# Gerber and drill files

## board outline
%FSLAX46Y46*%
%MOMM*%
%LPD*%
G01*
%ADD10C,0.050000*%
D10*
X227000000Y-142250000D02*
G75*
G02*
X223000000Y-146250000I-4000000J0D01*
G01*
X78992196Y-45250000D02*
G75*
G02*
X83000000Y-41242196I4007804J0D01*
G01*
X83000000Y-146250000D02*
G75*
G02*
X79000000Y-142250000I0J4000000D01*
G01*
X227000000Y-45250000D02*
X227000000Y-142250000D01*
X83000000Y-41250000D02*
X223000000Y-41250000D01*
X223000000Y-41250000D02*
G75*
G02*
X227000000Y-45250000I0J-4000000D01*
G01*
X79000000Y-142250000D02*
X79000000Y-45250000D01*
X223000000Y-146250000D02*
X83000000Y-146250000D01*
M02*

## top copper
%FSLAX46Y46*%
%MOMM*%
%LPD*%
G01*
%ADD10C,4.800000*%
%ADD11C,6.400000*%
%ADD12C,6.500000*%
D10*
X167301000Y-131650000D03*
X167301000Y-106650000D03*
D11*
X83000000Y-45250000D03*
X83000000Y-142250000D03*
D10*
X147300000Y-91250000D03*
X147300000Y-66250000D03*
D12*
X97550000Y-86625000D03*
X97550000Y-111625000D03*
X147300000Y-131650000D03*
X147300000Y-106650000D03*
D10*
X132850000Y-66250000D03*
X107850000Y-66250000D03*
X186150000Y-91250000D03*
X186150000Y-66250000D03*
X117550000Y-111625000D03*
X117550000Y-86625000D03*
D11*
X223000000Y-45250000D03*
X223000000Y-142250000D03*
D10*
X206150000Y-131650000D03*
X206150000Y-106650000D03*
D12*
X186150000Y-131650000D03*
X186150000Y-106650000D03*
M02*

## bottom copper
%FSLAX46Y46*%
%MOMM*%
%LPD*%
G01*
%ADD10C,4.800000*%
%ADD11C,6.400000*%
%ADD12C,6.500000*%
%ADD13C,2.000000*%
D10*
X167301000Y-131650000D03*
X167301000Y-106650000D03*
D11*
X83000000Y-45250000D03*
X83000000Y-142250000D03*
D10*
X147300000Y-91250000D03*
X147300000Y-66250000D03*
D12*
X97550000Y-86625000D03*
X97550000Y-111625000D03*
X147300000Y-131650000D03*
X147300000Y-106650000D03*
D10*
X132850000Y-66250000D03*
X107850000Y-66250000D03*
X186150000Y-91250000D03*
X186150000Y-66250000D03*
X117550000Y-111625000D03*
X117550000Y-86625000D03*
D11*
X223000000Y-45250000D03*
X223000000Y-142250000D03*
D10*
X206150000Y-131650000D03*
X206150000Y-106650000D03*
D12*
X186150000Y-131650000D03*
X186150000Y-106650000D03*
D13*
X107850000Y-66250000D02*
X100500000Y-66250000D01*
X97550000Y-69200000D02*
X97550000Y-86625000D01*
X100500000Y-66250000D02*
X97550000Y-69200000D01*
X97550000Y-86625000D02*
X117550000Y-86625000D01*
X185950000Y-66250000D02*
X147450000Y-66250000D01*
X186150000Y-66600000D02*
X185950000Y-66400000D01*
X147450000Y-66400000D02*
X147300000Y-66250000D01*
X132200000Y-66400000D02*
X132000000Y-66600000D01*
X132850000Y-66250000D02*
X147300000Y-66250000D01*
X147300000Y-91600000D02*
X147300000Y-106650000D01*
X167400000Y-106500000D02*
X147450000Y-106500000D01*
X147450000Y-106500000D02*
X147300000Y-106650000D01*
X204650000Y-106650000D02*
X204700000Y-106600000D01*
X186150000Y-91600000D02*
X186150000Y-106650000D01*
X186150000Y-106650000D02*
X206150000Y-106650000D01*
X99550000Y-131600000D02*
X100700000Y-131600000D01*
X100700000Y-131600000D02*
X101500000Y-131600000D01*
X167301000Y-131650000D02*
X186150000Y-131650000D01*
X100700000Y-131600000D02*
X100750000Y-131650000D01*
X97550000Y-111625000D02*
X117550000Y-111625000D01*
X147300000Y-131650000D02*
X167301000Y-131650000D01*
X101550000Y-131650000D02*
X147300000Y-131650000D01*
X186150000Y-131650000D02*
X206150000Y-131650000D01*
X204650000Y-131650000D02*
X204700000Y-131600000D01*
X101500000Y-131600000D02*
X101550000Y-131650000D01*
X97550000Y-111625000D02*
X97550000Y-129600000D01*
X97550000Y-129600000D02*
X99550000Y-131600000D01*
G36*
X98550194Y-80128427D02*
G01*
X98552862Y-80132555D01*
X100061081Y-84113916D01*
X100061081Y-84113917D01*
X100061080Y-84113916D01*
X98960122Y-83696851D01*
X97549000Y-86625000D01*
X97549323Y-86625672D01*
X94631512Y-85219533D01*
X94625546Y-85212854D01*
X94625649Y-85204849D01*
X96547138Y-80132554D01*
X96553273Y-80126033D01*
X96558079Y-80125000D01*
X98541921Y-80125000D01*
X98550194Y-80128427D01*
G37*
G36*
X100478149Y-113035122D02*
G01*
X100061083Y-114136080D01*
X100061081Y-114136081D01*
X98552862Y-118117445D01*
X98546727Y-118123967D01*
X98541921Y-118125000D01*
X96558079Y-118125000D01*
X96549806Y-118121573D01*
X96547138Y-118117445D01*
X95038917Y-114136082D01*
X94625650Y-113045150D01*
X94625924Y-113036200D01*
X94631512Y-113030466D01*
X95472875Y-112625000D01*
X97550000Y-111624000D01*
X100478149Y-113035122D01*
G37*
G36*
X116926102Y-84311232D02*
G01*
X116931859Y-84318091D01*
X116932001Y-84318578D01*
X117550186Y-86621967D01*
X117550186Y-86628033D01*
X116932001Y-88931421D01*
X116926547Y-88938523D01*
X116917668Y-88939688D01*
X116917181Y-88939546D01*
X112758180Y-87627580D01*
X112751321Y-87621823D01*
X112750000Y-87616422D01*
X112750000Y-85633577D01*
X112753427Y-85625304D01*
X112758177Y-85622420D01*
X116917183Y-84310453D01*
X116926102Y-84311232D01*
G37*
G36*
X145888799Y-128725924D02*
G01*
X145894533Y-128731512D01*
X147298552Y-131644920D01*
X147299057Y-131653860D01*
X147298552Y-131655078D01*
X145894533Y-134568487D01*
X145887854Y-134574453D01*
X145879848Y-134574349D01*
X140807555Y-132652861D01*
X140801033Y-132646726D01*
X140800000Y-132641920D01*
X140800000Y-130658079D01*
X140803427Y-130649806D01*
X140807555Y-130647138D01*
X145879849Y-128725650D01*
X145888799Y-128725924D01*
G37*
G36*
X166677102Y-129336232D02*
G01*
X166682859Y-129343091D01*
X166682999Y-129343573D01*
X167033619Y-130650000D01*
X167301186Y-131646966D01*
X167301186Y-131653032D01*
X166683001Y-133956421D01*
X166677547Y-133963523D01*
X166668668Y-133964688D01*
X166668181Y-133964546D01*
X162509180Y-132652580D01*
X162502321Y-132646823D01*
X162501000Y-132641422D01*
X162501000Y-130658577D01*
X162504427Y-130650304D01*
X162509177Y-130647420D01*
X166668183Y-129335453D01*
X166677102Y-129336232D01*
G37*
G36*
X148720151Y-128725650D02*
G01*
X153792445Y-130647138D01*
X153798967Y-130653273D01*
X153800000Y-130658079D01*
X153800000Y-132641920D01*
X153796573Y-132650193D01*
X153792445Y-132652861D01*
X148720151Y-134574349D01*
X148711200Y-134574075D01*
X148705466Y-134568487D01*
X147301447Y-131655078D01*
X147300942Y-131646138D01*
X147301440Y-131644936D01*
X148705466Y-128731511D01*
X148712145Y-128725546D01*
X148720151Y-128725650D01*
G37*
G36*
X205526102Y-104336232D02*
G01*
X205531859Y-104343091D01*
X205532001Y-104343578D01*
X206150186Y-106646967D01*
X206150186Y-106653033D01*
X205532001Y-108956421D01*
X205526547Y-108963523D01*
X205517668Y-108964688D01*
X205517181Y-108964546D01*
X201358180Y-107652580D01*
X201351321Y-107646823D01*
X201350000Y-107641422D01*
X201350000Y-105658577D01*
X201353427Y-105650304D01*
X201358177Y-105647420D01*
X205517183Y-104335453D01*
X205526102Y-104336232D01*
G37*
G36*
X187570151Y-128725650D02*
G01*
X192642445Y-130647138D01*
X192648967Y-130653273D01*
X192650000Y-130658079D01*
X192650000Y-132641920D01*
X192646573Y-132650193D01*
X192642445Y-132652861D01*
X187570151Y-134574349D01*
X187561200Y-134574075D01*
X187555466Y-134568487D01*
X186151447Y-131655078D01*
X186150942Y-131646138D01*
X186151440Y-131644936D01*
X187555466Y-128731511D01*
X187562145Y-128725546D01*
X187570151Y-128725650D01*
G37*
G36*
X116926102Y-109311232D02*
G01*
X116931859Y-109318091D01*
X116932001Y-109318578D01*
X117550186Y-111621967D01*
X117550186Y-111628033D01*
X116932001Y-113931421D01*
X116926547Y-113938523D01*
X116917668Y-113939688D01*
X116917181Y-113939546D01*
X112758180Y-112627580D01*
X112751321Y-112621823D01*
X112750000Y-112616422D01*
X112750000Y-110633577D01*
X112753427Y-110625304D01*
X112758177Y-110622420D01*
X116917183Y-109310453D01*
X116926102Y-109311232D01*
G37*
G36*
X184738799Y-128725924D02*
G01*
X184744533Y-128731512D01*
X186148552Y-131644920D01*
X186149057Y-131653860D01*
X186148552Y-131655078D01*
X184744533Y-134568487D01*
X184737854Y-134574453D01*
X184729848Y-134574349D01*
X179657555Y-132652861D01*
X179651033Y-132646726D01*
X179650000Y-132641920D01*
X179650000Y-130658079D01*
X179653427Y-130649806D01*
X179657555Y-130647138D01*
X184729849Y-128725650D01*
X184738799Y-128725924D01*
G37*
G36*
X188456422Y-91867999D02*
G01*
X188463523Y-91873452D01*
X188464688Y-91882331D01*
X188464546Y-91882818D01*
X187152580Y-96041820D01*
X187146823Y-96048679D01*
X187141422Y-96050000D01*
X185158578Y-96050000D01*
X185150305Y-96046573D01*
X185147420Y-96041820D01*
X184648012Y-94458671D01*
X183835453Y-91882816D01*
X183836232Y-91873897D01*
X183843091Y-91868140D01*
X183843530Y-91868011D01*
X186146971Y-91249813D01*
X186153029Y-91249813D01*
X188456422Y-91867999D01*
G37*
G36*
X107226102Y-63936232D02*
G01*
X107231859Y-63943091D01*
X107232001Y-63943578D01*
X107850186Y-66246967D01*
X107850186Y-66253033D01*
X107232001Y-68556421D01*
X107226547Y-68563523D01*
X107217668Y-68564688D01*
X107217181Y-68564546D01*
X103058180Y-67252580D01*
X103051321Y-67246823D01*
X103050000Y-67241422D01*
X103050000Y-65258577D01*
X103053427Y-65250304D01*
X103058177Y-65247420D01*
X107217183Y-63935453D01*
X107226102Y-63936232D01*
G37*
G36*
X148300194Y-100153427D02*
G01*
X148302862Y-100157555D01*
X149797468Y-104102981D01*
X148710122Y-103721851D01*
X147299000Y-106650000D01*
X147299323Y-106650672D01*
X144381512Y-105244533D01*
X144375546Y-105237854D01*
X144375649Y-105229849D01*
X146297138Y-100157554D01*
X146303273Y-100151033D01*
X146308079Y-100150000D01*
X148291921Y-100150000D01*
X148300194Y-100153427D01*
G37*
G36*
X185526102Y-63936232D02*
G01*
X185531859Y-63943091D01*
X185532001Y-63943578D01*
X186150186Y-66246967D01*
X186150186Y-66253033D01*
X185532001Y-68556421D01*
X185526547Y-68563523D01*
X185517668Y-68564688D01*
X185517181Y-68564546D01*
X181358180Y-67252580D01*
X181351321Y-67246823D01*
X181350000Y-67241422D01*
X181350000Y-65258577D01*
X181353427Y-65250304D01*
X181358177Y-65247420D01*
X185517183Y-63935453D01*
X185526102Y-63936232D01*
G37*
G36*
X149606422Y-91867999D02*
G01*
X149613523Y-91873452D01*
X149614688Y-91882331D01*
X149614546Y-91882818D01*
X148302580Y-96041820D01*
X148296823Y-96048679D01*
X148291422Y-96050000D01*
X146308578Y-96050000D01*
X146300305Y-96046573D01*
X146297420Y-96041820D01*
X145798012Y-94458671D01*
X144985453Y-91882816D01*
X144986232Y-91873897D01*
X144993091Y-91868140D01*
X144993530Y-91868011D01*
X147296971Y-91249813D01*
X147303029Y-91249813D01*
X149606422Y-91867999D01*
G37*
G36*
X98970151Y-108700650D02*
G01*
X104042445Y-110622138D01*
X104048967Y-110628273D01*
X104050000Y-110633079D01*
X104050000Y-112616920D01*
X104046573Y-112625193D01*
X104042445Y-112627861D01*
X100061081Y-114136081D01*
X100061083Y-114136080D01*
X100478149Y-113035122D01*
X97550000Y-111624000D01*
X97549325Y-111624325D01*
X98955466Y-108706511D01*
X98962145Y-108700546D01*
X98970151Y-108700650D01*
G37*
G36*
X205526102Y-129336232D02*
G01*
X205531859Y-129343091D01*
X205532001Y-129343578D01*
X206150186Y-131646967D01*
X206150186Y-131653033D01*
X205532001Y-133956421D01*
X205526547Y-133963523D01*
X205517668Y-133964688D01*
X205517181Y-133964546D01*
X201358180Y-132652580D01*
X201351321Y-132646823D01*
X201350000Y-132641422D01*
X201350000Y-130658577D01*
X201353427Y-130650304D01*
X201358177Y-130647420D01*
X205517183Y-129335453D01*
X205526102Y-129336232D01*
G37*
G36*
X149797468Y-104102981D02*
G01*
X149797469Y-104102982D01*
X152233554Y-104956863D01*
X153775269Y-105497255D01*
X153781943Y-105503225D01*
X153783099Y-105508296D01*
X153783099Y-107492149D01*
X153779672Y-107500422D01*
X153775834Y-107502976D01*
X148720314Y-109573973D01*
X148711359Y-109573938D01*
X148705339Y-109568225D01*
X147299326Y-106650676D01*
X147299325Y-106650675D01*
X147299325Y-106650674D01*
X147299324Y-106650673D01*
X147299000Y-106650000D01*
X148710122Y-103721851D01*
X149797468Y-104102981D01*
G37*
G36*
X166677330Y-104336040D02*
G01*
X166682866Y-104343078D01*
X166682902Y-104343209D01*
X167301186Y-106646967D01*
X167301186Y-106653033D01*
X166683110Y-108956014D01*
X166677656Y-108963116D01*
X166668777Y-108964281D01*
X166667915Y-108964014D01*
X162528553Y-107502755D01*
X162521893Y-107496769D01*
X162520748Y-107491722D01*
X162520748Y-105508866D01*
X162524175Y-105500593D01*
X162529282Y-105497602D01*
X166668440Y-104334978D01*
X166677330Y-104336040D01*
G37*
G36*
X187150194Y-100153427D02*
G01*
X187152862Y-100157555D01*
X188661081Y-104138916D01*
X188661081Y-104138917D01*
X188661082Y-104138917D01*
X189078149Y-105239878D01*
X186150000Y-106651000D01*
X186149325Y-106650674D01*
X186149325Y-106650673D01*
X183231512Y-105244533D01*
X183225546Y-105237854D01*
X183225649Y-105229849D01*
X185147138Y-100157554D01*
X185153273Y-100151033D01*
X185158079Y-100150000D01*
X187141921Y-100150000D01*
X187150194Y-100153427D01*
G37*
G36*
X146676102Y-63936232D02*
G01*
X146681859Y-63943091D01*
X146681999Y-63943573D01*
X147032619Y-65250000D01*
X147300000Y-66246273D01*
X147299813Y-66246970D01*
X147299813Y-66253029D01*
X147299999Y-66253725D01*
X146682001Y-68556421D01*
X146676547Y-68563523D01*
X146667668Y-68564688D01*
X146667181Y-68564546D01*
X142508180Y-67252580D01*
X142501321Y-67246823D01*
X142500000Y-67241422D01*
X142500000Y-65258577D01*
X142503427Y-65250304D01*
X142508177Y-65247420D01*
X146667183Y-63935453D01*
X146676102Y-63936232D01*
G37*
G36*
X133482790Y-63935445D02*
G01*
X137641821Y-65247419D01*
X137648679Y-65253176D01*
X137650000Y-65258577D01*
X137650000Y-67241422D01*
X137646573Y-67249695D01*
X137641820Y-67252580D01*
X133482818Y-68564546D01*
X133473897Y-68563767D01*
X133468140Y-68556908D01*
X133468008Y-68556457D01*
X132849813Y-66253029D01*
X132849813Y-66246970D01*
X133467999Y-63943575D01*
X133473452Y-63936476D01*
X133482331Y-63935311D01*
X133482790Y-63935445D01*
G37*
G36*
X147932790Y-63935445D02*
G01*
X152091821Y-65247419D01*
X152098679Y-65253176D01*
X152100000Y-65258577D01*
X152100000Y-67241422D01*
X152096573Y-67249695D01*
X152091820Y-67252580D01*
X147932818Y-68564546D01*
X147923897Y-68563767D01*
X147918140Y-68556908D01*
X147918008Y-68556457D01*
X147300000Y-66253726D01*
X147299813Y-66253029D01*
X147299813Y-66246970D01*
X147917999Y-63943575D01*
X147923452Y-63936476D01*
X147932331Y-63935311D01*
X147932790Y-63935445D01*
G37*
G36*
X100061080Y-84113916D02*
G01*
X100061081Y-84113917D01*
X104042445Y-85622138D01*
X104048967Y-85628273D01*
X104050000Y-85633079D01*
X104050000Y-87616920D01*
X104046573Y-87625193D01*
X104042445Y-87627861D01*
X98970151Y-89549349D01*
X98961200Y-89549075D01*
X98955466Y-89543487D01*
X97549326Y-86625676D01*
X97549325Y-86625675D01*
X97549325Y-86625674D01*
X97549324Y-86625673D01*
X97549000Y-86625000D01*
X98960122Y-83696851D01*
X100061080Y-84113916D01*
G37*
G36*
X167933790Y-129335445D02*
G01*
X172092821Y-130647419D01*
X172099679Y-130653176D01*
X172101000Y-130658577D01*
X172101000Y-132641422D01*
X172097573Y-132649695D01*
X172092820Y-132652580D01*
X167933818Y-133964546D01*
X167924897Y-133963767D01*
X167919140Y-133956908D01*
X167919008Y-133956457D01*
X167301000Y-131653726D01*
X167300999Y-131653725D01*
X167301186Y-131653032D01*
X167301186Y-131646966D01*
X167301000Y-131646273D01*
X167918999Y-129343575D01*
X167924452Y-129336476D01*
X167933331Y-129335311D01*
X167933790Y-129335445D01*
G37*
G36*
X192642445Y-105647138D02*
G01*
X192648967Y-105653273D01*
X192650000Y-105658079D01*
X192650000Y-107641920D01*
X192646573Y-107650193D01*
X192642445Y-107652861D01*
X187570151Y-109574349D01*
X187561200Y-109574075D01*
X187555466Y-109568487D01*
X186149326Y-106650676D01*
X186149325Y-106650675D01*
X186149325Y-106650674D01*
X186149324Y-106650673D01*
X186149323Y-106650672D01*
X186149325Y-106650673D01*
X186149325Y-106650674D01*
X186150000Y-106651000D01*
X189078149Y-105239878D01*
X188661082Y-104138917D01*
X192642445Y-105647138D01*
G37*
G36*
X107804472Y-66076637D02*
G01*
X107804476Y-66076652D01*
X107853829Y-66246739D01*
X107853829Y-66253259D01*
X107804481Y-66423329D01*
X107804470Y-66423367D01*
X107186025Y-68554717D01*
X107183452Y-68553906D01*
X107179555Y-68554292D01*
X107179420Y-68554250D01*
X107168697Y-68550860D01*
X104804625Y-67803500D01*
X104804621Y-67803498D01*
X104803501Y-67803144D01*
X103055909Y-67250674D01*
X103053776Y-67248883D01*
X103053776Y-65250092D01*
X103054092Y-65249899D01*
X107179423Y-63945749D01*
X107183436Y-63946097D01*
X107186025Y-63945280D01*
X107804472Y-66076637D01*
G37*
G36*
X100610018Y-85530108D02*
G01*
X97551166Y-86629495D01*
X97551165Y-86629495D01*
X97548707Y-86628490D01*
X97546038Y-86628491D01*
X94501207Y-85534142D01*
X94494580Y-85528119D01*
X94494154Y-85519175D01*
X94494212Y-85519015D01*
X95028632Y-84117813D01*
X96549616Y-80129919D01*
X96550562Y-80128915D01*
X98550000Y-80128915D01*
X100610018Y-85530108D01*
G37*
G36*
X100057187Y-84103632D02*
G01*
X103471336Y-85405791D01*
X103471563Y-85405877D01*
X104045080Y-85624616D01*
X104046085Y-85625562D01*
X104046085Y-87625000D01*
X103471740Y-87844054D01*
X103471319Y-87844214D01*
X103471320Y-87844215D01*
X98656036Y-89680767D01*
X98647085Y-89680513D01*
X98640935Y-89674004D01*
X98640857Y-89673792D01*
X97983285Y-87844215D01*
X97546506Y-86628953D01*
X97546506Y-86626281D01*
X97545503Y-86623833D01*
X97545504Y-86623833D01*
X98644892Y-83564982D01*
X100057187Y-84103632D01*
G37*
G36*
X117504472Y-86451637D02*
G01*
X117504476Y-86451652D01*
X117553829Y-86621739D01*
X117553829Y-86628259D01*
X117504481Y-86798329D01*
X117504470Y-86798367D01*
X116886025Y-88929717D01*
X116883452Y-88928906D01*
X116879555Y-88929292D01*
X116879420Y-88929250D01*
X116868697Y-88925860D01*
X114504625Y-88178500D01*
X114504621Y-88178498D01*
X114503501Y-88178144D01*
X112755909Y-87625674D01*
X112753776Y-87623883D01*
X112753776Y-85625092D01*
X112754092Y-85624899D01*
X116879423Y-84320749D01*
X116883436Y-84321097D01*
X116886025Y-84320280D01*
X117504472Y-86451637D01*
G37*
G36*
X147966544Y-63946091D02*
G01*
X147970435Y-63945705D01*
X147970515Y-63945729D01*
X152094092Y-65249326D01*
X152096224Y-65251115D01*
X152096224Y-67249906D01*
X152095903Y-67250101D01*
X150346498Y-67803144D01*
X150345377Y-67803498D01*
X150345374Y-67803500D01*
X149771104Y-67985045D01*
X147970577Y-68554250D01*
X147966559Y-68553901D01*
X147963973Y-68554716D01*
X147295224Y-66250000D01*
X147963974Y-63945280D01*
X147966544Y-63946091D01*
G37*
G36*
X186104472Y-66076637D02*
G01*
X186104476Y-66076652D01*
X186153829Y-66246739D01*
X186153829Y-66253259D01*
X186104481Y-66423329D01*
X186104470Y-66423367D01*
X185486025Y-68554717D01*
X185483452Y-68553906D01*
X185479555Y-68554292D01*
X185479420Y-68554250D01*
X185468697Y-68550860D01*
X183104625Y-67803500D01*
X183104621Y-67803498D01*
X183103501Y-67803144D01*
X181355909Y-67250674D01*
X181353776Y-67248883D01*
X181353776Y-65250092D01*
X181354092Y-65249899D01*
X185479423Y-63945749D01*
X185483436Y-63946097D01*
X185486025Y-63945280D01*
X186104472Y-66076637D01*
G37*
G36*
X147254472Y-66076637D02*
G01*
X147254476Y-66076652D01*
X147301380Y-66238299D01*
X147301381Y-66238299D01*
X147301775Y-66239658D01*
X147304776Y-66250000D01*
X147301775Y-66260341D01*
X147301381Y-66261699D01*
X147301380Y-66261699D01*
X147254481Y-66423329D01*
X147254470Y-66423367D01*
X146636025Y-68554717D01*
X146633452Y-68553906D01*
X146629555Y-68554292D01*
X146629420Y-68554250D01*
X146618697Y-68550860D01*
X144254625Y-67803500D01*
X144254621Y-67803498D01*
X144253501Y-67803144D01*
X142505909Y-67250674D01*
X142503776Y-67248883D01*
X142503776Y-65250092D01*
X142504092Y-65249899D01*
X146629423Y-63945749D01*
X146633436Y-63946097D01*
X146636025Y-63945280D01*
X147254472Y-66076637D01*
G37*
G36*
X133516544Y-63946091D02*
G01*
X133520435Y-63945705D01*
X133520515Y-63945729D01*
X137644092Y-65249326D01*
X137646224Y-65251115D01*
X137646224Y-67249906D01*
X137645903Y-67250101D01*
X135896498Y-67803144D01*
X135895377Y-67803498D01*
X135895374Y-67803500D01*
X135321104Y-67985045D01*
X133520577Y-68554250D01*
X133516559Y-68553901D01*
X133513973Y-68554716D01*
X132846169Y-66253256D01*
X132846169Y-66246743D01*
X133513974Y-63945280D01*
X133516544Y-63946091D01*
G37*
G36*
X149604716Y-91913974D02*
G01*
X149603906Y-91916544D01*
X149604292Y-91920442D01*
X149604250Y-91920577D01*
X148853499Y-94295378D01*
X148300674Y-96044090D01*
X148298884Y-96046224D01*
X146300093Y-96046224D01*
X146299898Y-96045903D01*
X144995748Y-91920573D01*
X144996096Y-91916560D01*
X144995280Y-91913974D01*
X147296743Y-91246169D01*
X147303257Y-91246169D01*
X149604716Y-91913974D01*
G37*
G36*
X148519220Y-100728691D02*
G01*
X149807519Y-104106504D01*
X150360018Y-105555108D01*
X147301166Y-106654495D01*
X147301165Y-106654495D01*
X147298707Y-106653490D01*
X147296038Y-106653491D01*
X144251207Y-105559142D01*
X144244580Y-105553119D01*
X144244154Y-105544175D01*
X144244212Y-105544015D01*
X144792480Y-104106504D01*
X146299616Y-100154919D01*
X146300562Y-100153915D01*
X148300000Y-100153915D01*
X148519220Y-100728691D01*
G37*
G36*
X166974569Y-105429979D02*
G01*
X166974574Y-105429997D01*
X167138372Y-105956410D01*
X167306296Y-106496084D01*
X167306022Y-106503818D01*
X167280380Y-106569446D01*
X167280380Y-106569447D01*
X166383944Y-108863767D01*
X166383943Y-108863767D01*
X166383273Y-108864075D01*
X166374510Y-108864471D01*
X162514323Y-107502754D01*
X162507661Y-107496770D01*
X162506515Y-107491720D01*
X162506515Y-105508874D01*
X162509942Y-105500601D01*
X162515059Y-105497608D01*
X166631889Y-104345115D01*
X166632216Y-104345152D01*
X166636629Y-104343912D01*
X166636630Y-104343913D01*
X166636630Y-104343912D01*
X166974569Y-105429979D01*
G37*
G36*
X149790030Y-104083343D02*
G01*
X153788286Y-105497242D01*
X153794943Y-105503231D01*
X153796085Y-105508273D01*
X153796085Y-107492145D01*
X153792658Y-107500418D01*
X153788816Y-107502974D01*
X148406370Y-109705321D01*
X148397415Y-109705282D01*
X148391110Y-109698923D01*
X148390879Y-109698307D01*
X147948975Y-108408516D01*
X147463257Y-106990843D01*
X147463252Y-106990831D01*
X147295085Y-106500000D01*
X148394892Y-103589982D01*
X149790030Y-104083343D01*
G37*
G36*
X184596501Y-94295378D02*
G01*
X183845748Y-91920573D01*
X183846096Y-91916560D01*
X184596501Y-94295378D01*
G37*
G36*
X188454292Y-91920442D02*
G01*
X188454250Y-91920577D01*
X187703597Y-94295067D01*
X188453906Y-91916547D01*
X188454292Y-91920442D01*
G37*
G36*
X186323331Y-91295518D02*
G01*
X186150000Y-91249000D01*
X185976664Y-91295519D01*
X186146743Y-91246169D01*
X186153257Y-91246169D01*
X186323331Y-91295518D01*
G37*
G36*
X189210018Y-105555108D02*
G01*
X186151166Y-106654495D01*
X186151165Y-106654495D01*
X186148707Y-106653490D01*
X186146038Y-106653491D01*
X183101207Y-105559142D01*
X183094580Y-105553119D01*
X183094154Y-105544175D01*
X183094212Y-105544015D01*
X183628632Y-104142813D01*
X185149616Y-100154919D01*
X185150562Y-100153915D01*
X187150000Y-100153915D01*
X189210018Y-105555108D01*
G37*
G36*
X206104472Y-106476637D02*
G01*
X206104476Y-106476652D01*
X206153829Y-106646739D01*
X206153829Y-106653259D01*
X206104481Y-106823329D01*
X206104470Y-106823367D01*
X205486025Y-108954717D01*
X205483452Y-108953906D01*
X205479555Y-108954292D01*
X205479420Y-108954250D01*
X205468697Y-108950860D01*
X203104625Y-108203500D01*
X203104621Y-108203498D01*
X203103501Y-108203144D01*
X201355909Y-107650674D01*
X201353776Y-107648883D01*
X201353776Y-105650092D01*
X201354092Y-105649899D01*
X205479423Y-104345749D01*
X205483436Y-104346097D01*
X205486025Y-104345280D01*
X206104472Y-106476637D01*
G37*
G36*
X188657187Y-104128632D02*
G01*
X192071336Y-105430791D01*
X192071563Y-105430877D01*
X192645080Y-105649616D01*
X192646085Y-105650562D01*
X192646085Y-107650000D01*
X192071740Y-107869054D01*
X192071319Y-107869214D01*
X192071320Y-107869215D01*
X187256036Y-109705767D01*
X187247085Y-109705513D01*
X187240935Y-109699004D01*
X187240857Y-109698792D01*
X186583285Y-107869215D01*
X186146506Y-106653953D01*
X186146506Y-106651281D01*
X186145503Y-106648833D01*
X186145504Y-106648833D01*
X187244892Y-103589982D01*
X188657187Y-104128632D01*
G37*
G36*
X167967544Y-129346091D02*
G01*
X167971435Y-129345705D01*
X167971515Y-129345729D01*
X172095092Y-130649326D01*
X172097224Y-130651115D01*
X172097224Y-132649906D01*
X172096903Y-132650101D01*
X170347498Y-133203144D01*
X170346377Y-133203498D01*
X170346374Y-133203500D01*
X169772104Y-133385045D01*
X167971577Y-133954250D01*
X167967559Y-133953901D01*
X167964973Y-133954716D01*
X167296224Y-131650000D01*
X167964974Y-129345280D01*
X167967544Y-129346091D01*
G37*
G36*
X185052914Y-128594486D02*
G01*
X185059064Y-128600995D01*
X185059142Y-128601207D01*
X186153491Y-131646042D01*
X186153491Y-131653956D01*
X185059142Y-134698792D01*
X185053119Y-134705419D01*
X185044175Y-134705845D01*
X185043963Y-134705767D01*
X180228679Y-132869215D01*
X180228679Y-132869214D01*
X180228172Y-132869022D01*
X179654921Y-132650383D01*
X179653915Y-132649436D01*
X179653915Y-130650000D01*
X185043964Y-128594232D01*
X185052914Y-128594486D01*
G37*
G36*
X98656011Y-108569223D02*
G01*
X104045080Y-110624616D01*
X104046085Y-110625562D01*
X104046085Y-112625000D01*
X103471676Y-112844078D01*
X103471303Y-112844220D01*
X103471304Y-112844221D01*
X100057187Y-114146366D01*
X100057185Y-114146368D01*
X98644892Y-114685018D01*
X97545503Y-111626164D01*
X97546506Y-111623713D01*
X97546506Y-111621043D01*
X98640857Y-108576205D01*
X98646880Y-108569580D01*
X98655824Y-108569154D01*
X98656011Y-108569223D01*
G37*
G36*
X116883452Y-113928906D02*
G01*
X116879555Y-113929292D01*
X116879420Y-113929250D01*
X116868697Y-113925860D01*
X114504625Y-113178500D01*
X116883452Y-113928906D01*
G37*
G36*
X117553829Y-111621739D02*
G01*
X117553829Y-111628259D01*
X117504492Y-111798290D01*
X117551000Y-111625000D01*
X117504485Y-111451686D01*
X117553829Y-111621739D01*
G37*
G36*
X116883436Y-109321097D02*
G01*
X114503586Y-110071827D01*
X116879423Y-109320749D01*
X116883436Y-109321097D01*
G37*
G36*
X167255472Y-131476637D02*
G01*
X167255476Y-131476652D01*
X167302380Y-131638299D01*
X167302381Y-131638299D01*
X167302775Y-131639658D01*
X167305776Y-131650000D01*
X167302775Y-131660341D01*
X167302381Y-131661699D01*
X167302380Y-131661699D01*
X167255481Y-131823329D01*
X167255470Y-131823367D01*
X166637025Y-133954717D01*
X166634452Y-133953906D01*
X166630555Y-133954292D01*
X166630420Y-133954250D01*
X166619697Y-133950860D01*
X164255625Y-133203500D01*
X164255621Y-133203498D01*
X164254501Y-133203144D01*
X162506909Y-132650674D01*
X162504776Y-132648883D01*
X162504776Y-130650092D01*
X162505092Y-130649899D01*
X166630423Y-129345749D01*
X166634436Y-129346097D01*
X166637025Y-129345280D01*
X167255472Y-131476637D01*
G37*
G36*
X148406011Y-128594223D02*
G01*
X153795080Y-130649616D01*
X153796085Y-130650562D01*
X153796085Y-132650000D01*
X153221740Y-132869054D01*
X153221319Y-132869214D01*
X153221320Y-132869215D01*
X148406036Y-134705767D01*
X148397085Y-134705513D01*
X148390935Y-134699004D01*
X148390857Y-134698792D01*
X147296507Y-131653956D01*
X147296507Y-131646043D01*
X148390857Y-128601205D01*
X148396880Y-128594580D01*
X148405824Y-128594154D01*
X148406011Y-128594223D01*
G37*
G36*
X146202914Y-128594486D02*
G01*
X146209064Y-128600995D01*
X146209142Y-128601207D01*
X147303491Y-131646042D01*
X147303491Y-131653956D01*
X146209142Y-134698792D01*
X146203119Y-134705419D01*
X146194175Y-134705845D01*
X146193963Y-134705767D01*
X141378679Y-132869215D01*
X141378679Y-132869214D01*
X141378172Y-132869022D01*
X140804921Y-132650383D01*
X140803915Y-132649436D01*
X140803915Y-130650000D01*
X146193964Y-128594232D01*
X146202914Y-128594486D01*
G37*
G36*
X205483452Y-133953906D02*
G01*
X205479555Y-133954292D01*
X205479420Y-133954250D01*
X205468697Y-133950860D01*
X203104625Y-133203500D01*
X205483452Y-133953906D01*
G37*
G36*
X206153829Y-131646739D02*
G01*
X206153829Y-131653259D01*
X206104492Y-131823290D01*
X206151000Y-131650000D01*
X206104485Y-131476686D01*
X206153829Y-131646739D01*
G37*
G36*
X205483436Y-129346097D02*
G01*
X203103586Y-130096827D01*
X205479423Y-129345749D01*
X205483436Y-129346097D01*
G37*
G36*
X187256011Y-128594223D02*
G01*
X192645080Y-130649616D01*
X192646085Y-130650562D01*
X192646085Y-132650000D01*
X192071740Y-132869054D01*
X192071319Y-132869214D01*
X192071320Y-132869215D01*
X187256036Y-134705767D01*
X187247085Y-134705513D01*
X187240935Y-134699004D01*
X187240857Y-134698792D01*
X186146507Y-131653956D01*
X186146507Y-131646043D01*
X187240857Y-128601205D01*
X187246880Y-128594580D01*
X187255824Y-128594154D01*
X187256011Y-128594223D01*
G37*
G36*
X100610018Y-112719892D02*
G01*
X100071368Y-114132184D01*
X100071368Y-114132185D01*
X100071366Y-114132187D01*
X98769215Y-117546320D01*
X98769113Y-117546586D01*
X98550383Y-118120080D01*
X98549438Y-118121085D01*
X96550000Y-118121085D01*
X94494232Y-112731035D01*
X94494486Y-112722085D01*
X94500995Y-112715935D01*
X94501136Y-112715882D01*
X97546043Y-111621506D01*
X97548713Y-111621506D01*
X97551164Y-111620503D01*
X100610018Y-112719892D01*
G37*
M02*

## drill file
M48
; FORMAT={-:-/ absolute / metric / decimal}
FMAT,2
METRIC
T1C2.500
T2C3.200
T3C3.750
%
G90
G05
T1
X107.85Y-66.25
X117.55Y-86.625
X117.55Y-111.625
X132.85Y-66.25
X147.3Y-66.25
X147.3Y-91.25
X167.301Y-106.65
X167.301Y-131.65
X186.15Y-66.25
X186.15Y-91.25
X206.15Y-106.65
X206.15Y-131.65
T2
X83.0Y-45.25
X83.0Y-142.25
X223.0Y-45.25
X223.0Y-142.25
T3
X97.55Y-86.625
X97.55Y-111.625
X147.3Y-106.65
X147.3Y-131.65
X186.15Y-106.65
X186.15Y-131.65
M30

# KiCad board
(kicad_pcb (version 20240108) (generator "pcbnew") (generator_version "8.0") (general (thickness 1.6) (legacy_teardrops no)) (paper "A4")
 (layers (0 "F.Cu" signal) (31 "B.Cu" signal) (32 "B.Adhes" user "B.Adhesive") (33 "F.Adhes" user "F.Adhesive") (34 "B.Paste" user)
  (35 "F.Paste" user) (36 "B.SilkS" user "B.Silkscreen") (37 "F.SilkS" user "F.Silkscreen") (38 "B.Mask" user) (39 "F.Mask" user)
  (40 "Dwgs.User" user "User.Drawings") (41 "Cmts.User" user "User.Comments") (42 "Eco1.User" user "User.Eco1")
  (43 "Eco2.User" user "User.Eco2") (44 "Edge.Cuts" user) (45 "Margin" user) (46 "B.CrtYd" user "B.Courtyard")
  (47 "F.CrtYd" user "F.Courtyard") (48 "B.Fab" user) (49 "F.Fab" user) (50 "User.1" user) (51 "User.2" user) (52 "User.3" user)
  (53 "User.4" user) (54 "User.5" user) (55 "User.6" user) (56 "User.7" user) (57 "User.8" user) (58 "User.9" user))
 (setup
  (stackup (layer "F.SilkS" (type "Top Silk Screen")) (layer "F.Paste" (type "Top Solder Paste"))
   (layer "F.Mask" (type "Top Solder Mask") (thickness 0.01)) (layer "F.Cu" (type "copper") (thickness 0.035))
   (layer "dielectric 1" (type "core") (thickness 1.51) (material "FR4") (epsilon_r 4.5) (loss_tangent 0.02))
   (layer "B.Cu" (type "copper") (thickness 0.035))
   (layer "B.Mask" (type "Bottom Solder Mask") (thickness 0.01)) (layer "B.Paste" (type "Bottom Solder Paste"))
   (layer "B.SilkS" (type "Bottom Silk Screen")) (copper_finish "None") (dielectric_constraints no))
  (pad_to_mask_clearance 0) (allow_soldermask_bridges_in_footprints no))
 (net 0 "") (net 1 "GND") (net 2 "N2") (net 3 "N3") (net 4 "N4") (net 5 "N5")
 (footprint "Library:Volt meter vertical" (layer "F.Cu") (at 167.301 119.15)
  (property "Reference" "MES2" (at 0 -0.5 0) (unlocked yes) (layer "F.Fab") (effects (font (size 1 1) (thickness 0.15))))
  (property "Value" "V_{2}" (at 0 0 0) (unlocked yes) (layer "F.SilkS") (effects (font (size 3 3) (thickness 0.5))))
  (pad "1" thru_hole circle (at 0 12.5 180) (size 4.8 4.8) (drill 2.5) (layers "*.Cu" "*.Mask") (remove_unused_layers no) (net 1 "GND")
   (teardrops (best_length_ratio 0.5) (max_length 8) (best_width_ratio 1) (max_width 8) (curve_points 0) (filter_ratio 0.9) (enabled yes)
    (allow_two_segments yes) (prefer_zone_connections yes)))
  (pad "2" thru_hole circle (at 0 -12.5 180) (size 4.8 4.8) (drill 2.5) (layers "*.Cu" "*.Mask") (remove_unused_layers no) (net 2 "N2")
   (teardrops (best_length_ratio 0.5) (max_length 8) (best_width_ratio 1) (max_width 8) (curve_points 0) (filter_ratio 0.9) (enabled yes)
    (allow_two_segments yes) (prefer_zone_connections yes))))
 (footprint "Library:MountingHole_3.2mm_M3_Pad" (layer "F.Cu") (at 83 45.25)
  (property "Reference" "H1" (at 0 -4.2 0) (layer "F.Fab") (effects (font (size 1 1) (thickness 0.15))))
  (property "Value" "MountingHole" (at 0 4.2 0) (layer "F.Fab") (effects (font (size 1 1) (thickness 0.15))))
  (pad "1" thru_hole circle (at 0 0) (size 6.4 6.4) (drill 3.2) (layers "*.Cu" "*.Mask") (remove_unused_layers no)))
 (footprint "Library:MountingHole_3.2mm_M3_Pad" (layer "F.Cu") (at 83 142.25)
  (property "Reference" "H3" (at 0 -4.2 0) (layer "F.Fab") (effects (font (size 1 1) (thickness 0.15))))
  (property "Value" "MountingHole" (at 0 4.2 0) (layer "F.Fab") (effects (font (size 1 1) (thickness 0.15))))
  (pad "1" thru_hole circle (at 0 0) (size 6.4 6.4) (drill 3.2) (layers "*.Cu" "*.Mask") (remove_unused_layers no)))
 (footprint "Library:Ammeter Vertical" (layer "F.Cu") (at 147.3 78.75 -90)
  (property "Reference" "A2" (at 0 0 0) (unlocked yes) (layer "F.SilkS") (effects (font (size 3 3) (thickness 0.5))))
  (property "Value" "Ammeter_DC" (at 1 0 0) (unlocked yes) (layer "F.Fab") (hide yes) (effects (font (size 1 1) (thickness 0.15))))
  (pad "1" thru_hole circle (at 12.5 0 180) (size 4.8 4.8) (drill 2.5) (layers "*.Cu" "*.Mask") (remove_unused_layers no) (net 2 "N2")
   (teardrops (best_length_ratio 0.5) (max_length 8) (best_width_ratio 1) (max_width 8) (curve_points 0) (filter_ratio 0.9) (enabled yes)
    (allow_two_segments yes) (prefer_zone_connections yes)))
  (pad "2" thru_hole circle (at -12.5 0 180) (size 4.8 4.8) (drill 2.5) (layers "*.Cu" "*.Mask") (remove_unused_layers no) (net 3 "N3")
   (teardrops (best_length_ratio 0.5) (max_length 8) (best_width_ratio 1) (max_width 8) (curve_points 0) (filter_ratio 0.9) (enabled yes)
    (allow_two_segments yes) (prefer_zone_connections yes))))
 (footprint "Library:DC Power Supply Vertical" (layer "F.Cu") (at 97.55 99.125)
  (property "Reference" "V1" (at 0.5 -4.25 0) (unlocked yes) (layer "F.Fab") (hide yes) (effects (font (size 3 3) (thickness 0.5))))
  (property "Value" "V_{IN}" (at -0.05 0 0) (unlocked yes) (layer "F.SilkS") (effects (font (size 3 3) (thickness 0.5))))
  (pad "1" thru_hole circle (at 0 -12.5) (size 6.5 6.5) (drill 3.75) (layers "*.Cu" "*.Mask") (remove_unused_layers no) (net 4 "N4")
   (teardrops (best_length_ratio 0.5) (max_length 8) (best_width_ratio 1) (max_width 8) (curve_points 0) (filter_ratio 0.9) (enabled yes)
    (allow_two_segments yes) (prefer_zone_connections yes)))
  (pad "2" thru_hole circle (at 0 12.5) (size 6.5 6.5) (drill 3.75) (layers "*.Cu" "*.Mask") (remove_unused_layers no) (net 1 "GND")
   (teardrops (best_length_ratio 0.5) (max_length 8) (best_width_ratio 1) (max_width 8) (curve_points 0) (filter_ratio 0.9) (enabled yes)
    (allow_two_segments yes) (prefer_zone_connections yes))))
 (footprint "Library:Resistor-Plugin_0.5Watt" (layer "F.Cu") (at 147.3 119.15 180)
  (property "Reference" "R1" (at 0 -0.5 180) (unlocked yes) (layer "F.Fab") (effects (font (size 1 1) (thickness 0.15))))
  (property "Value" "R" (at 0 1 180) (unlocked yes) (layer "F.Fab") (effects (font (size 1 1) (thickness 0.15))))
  (pad "1" thru_hole circle (at 0 -12.5 180) (size 6.5 6.5) (drill 3.75) (layers "*.Cu" "*.Mask") (remove_unused_layers no) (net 1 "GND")
   (teardrops (best_length_ratio 0.5) (max_length 8) (best_width_ratio 1) (max_width 8) (curve_points 0) (filter_ratio 0.9) (enabled yes)
    (allow_two_segments yes) (prefer_zone_connections yes)))
  (pad "2" thru_hole circle (at 0 12.5 180) (size 6.5 6.5) (drill 3.75) (layers "*.Cu" "*.Mask") (remove_unused_layers no) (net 2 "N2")
   (teardrops (best_length_ratio 0.5) (max_length 8) (best_width_ratio 1) (max_width 8) (curve_points 0) (filter_ratio 0.9) (enabled yes)
    (allow_two_segments yes) (prefer_zone_connections yes))))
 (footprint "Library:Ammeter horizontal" (layer "F.Cu") (at 120.35 66.25)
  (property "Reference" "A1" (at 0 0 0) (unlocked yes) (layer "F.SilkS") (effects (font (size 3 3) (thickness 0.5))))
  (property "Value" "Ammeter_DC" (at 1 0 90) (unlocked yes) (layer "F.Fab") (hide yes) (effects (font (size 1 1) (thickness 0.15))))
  (pad "1" thru_hole circle (at 12.5 0 270) (size 4.8 4.8) (drill 2.5) (layers "*.Cu" "*.Mask") (remove_unused_layers no) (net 3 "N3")
   (teardrops (best_length_ratio 0.5) (max_length 8) (best_width_ratio 1) (max_width 8) (curve_points 0) (filter_ratio 0.9) (enabled yes)
    (allow_two_segments yes) (prefer_zone_connections yes)))
  (pad "2" thru_hole circle (at -12.5 0 270) (size 4.8 4.8) (drill 2.5) (layers "*.Cu" "*.Mask") (remove_unused_layers no) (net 4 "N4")
   (teardrops (best_length_ratio 0.5) (max_length 8) (best_width_ratio 1) (max_width 8) (curve_points 0) (filter_ratio 0.9) (enabled yes)
    (allow_two_segments yes) (prefer_zone_connections yes))))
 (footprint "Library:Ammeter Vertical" (layer "F.Cu") (at 186.15 78.75 -90)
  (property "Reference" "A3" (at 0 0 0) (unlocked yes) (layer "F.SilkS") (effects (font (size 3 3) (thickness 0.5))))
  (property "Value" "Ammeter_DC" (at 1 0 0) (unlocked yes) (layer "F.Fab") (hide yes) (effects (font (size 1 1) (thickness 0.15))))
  (pad "1" thru_hole circle (at 12.5 0 180) (size 4.8 4.8) (drill 2.5) (layers "*.Cu" "*.Mask") (remove_unused_layers no) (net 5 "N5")
   (teardrops (best_length_ratio 0.5) (max_length 8) (best_width_ratio 1) (max_width 8) (curve_points 0) (filter_ratio 0.9) (enabled yes)
    (allow_two_segments yes) (prefer_zone_connections yes)))
  (pad "2" thru_hole circle (at -12.5 0 180) (size 4.8 4.8) (drill 2.5) (layers "*.Cu" "*.Mask") (remove_unused_layers no) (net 3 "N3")
   (teardrops (best_length_ratio 0.5) (max_length 8) (best_width_ratio 1) (max_width 8) (curve_points 0) (filter_ratio 0.9) (enabled yes)
    (allow_two_segments yes) (prefer_zone_connections yes))))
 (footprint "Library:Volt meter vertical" (layer "F.Cu") (at 117.55 99.125)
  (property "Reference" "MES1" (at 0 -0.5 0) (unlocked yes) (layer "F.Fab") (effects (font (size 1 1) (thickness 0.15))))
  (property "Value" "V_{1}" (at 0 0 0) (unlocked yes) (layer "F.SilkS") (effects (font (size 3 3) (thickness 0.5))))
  (pad "1" thru_hole circle (at 0 12.5 180) (size 4.8 4.8) (drill 2.5) (layers "*.Cu" "*.Mask") (remove_unused_layers no) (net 1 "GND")
   (teardrops (best_length_ratio 0.5) (max_length 8) (best_width_ratio 1) (max_width 8) (curve_points 0) (filter_ratio 0.9) (enabled yes)
    (allow_two_segments yes) (prefer_zone_connections yes)))
  (pad "2" thru_hole circle (at 0 -12.5 180) (size 4.8 4.8) (drill 2.5) (layers "*.Cu" "*.Mask") (remove_unused_layers no) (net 4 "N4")
   (teardrops (best_length_ratio 0.5) (max_length 8) (best_width_ratio 1) (max_width 8) (curve_points 0) (filter_ratio 0.9) (enabled yes)
    (allow_two_segments yes) (prefer_zone_connections yes))))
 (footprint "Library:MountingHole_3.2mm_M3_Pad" (layer "F.Cu") (at 223 45.25)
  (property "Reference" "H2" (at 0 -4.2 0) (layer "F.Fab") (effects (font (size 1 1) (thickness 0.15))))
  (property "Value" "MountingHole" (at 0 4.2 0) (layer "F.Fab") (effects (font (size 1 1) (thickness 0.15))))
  (pad "1" thru_hole circle (at 0 0) (size 6.4 6.4) (drill 3.2) (layers "*.Cu" "*.Mask") (remove_unused_layers no)))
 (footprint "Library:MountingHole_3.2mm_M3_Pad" (layer "F.Cu") (at 223 142.25)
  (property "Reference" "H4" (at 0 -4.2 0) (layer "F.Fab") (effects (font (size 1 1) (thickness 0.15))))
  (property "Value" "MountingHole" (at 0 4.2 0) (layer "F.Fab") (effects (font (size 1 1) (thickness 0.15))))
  (pad "1" thru_hole circle (at 0 0) (size 6.4 6.4) (drill 3.2) (layers "*.Cu" "*.Mask") (remove_unused_layers no)))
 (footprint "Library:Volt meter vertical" (layer "F.Cu") (at 206.15 119.15)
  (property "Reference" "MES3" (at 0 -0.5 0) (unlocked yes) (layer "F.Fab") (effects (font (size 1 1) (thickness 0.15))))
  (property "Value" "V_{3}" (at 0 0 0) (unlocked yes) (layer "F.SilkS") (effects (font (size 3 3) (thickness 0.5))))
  (pad "1" thru_hole circle (at 0 12.5 180) (size 4.8 4.8) (drill 2.5) (layers "*.Cu" "*.Mask") (remove_unused_layers no) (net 1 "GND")
   (teardrops (best_length_ratio 0.5) (max_length 8) (best_width_ratio 1) (max_width 8) (curve_points 0) (filter_ratio 0.9) (enabled yes)
    (allow_two_segments yes) (prefer_zone_connections yes)))
  (pad "2" thru_hole circle (at 0 -12.5 180) (size 4.8 4.8) (drill 2.5) (layers "*.Cu" "*.Mask") (remove_unused_layers no) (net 5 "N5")
   (teardrops (best_length_ratio 0.5) (max_length 8) (best_width_ratio 1) (max_width 8) (curve_points 0) (filter_ratio 0.9) (enabled yes)
    (allow_two_segments yes) (prefer_zone_connections yes))))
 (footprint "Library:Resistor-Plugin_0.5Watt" (layer "F.Cu") (at 186.15 119.15 180)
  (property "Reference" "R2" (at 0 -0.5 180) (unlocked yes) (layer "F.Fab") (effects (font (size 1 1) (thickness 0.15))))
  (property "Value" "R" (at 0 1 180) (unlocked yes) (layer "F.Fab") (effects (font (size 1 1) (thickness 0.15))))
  (pad "1" thru_hole circle (at 0 -12.5 180) (size 6.5 6.5) (drill 3.75) (layers "*.Cu" "*.Mask") (remove_unused_layers no) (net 1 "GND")
   (teardrops (best_length_ratio 0.5) (max_length 8) (best_width_ratio 1) (max_width 8) (curve_points 0) (filter_ratio 0.9) (enabled yes)
    (allow_two_segments yes) (prefer_zone_connections yes)))
  (pad "2" thru_hole circle (at 0 12.5 180) (size 6.5 6.5) (drill 3.75) (layers "*.Cu" "*.Mask") (remove_unused_layers no) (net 5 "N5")
   (teardrops (best_length_ratio 0.5) (max_length 8) (best_width_ratio 1) (max_width 8) (curve_points 0) (filter_ratio 0.9) (enabled yes)
    (allow_two_segments yes) (prefer_zone_connections yes))))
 (gr_arc (start 227 142.25) (mid 225.828427 145.078427) (end 223 146.25) (stroke (width 0.05) (type default)) (layer "Edge.Cuts"))
 (gr_arc (start 78.992196 45.25) (mid 80.166055 42.416055) (end 83 41.242196) (stroke (width 0.05) (type default)) (layer "Edge.Cuts"))
 (gr_arc (start 83 146.25) (mid 80.171573 145.078427) (end 79 142.25) (stroke (width 0.05) (type default)) (layer "Edge.Cuts"))
 (gr_line (start 227 45.25) (end 227 142.25) (stroke (width 0.05) (type default)) (layer "Edge.Cuts"))
 (gr_line (start 83 41.25) (end 223 41.25) (locked yes) (stroke (width 0.05) (type default)) (layer "Edge.Cuts"))
 (gr_arc (start 223 41.25) (mid 225.828427 42.421573) (end 227 45.25) (stroke (width 0.05) (type default)) (layer "Edge.Cuts"))
 (gr_line (start 79 142.25) (end 79 45.25) (stroke (width 0.05) (type default)) (layer "Edge.Cuts"))
 (gr_line (start 223 146.25) (end 83 146.25) (stroke (width 0.05) (type default)) (layer "Edge.Cuts"))
 (segment (start 107.85 66.25) (end 100.5 66.25) (width 2) (layer "B.Cu") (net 4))
 (segment (start 97.55 69.2) (end 97.55 86.625) (width 2) (layer "B.Cu") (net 4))
 (segment (start 100.5 66.25) (end 97.55 69.2) (width 2) (layer "B.Cu") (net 4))
 (segment (start 97.55 86.625) (end 117.55 86.625) (width 2) (layer "B.Cu") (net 4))
 (segment (start 185.95 66.25) (end 147.45 66.25) (width 2) (layer "B.Cu") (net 3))
 (segment (start 186.15 66.6) (end 185.95 66.4) (width 2) (layer "B.Cu") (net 3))
 (segment (start 147.45 66.4) (end 147.3 66.25) (width 2) (layer "B.Cu") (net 3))
 (segment (start 132.2 66.4) (end 132 66.6) (width 2) (layer "B.Cu") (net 3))
 (segment (start 132.85 66.25) (end 147.3 66.25) (width 2) (layer "B.Cu") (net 3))
 (segment (start 147.3 91.6) (end 147.3 106.65) (width 2) (layer "B.Cu") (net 2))
 (segment (start 167.4 106.5) (end 147.45 106.5) (width 2) (layer "B.Cu") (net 2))
 (segment (start 147.45 106.5) (end 147.3 106.65) (width 2) (layer "B.Cu") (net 2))
 (segment (start 204.65 106.65) (end 204.7 106.6) (width 2) (layer "B.Cu") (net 5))
 (segment (start 186.15 91.6) (end 186.15 106.65) (width 2) (layer "B.Cu") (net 5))
 (segment (start 186.15 106.65) (end 206.15 106.65) (width 2) (layer "B.Cu") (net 5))
 (segment (start 99.55 131.6) (end 100.7 131.6) (width 2) (layer "B.Cu") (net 1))
 (segment (start 100.7 131.6) (end 101.5 131.6) (width 2) (layer "B.Cu") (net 1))
 (segment (start 167.301 131.65) (end 186.15 131.65) (width 2) (layer "B.Cu") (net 1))
 (segment (start 100.7 131.6) (end 100.75 131.65) (width 2) (layer "B.Cu") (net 1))
 (segment (start 97.55 111.625) (end 117.55 111.625) (width 2) (layer "B.Cu") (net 1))
 (segment (start 147.3 131.65) (end 167.301 131.65) (width 2) (layer "B.Cu") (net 1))
 (segment (start 101.55 131.65) (end 147.3 131.65) (width 2) (layer "B.Cu") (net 1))
 (segment (start 186.15 131.65) (end 206.15 131.65) (width 2) (layer "B.Cu") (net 1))
 (segment (start 204.65 131.65) (end 204.7 131.6) (width 2) (layer "B.Cu") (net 1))
 (segment (start 101.5 131.6) (end 101.55 131.65) (width 2) (layer "B.Cu") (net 1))
 (segment (start 97.55 111.625) (end 97.55 129.6) (width 2) (layer "B.Cu") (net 1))
 (segment (start 97.55 129.6) (end 99.55 131.6) (width 2) (layer "B.Cu") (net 1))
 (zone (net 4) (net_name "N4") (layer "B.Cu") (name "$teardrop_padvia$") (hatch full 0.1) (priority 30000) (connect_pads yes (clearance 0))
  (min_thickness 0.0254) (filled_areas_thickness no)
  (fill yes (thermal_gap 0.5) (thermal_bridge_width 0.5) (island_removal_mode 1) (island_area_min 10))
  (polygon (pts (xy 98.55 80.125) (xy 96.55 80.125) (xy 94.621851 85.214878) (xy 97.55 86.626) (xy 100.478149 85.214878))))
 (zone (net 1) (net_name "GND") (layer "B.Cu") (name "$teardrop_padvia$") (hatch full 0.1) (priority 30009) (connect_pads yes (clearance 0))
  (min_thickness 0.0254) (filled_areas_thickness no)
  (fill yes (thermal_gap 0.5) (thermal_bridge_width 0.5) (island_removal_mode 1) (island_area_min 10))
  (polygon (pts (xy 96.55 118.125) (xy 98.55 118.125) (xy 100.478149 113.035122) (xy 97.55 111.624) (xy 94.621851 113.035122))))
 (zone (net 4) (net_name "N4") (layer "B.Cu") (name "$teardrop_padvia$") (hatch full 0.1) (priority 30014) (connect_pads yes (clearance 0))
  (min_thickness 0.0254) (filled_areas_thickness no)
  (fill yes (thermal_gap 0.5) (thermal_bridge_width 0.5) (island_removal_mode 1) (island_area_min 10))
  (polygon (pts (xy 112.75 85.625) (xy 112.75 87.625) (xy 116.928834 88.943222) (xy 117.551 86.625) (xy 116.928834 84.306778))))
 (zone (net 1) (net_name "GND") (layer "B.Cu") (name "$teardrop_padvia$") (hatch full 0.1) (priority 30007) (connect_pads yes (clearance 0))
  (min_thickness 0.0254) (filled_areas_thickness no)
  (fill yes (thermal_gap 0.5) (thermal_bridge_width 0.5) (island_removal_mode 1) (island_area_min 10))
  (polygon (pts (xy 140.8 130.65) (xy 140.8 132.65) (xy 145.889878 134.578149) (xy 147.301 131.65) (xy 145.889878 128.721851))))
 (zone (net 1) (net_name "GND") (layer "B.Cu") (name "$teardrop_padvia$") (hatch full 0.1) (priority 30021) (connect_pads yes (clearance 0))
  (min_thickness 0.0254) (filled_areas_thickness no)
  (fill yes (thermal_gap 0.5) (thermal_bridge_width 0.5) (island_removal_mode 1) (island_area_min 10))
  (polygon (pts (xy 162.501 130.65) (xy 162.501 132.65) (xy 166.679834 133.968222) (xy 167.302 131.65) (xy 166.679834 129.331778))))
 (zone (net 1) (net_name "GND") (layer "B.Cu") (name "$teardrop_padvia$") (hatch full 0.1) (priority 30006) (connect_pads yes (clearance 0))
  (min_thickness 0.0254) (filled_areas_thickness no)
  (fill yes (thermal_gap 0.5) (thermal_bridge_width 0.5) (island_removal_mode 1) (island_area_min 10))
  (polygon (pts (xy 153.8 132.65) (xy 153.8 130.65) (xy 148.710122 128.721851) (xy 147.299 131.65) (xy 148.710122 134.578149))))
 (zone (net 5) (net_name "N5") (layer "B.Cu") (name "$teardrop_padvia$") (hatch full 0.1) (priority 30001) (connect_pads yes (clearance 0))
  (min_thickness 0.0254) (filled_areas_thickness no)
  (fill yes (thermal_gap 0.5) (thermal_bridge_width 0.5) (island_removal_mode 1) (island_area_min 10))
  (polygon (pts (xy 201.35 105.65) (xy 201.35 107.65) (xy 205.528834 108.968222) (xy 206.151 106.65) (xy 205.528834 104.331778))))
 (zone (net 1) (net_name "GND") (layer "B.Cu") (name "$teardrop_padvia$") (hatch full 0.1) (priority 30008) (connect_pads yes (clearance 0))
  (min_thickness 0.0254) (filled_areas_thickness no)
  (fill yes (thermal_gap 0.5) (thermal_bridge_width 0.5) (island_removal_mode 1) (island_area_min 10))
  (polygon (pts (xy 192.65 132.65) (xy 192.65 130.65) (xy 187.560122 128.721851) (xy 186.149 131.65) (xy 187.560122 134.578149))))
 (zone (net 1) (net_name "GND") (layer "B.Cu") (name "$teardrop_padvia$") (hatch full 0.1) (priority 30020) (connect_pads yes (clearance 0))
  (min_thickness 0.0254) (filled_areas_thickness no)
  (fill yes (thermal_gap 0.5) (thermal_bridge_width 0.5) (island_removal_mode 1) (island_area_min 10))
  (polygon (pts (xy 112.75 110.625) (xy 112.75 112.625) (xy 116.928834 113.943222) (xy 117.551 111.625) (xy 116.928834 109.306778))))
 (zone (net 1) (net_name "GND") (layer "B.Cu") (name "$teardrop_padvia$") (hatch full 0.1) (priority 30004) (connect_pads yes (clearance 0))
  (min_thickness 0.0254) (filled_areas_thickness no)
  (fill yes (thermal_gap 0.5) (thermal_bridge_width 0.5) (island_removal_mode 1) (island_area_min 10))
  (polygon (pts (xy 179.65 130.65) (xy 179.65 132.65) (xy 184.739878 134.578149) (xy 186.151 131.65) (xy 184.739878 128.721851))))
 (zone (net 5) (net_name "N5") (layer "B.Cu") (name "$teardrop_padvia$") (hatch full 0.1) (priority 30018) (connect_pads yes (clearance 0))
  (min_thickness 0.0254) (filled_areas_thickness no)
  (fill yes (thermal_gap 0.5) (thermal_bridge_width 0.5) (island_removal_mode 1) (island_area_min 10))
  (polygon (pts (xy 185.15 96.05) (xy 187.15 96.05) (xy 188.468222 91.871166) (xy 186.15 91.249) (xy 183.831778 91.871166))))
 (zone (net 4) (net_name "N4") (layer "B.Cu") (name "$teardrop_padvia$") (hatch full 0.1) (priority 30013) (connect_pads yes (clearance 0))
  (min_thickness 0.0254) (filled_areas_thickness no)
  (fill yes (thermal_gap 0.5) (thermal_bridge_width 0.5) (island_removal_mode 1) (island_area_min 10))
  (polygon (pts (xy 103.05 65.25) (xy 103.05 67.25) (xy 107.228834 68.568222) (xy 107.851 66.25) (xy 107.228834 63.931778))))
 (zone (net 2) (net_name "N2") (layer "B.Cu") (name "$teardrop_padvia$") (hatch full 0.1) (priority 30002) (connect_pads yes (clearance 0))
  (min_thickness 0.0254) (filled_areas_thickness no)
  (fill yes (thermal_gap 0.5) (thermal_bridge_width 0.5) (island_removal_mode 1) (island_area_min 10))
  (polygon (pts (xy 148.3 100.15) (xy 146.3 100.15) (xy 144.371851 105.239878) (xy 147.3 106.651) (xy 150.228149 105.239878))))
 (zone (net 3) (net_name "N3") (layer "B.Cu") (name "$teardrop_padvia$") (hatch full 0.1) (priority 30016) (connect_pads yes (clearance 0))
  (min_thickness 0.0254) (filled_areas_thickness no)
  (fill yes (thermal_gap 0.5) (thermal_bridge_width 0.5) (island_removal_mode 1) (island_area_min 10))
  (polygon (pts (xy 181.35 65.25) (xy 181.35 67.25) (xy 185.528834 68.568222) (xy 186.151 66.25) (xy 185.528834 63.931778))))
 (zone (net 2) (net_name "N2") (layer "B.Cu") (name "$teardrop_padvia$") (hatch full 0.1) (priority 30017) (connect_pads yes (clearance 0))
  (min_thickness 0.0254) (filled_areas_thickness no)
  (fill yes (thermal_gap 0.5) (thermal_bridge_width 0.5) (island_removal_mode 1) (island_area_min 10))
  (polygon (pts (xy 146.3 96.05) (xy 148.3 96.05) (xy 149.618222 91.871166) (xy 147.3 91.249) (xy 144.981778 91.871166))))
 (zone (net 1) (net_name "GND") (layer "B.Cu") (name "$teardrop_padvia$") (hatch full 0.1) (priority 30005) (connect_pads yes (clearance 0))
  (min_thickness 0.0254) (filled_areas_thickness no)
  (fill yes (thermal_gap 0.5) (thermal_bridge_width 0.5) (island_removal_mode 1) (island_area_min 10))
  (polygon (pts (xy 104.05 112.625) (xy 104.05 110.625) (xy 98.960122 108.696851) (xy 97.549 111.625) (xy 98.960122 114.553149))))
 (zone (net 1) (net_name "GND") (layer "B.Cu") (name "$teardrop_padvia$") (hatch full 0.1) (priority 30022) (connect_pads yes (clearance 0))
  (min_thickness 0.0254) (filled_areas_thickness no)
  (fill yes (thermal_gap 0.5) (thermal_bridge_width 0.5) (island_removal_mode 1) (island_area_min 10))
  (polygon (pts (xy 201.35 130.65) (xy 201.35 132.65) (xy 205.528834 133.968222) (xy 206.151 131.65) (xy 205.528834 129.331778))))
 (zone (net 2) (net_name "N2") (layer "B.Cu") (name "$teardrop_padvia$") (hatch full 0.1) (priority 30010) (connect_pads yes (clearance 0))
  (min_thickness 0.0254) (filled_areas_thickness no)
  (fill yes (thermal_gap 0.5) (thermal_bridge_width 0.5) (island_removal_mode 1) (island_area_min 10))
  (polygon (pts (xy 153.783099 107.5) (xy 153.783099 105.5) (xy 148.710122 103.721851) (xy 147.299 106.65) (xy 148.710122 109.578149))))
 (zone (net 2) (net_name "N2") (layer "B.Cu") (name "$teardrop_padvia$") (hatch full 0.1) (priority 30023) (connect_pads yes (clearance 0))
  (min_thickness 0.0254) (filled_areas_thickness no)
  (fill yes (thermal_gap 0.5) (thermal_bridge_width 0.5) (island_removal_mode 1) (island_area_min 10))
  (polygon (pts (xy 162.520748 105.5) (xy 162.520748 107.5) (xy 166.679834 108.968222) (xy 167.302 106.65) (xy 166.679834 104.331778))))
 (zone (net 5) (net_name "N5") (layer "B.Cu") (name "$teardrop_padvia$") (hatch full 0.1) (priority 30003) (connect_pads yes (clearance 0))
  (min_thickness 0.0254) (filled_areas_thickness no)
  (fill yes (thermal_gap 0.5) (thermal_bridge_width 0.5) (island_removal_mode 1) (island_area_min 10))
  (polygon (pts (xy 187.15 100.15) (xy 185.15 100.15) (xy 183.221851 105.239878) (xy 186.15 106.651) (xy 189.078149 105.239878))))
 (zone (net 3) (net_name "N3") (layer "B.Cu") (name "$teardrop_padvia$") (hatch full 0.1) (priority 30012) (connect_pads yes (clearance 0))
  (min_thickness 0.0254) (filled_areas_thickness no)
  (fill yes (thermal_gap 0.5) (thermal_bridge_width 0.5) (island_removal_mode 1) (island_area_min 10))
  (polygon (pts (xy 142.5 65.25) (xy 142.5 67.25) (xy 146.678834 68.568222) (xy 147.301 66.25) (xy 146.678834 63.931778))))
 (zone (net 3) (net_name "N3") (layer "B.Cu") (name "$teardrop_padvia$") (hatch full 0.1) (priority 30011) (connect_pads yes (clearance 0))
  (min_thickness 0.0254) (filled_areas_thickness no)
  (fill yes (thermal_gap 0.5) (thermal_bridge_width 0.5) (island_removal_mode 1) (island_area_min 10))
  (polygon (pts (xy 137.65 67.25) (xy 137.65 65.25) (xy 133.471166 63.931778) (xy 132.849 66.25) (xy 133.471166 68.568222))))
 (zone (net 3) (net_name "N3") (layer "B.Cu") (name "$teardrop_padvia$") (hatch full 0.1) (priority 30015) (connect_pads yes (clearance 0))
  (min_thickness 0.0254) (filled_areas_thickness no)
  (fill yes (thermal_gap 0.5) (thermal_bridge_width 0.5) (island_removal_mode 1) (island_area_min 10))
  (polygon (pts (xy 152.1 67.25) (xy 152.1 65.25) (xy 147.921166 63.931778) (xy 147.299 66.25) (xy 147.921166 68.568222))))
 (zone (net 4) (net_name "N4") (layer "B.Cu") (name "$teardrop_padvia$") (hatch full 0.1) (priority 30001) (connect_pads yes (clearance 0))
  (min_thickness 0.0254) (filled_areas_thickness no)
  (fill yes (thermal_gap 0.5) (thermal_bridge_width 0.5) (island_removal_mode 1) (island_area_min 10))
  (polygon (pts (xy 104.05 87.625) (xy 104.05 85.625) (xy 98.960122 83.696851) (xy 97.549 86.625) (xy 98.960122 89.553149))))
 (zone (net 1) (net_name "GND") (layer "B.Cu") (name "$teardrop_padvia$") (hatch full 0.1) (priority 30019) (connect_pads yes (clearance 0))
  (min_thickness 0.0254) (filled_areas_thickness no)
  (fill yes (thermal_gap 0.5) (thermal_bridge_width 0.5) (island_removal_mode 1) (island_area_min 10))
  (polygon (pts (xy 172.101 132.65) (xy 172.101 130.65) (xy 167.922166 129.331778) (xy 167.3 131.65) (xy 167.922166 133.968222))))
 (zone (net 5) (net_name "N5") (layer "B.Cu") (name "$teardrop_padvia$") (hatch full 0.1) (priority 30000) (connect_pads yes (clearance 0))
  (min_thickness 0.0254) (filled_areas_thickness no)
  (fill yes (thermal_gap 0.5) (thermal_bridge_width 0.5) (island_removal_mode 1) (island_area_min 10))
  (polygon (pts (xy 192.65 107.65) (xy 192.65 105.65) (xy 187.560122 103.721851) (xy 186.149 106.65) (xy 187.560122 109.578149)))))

